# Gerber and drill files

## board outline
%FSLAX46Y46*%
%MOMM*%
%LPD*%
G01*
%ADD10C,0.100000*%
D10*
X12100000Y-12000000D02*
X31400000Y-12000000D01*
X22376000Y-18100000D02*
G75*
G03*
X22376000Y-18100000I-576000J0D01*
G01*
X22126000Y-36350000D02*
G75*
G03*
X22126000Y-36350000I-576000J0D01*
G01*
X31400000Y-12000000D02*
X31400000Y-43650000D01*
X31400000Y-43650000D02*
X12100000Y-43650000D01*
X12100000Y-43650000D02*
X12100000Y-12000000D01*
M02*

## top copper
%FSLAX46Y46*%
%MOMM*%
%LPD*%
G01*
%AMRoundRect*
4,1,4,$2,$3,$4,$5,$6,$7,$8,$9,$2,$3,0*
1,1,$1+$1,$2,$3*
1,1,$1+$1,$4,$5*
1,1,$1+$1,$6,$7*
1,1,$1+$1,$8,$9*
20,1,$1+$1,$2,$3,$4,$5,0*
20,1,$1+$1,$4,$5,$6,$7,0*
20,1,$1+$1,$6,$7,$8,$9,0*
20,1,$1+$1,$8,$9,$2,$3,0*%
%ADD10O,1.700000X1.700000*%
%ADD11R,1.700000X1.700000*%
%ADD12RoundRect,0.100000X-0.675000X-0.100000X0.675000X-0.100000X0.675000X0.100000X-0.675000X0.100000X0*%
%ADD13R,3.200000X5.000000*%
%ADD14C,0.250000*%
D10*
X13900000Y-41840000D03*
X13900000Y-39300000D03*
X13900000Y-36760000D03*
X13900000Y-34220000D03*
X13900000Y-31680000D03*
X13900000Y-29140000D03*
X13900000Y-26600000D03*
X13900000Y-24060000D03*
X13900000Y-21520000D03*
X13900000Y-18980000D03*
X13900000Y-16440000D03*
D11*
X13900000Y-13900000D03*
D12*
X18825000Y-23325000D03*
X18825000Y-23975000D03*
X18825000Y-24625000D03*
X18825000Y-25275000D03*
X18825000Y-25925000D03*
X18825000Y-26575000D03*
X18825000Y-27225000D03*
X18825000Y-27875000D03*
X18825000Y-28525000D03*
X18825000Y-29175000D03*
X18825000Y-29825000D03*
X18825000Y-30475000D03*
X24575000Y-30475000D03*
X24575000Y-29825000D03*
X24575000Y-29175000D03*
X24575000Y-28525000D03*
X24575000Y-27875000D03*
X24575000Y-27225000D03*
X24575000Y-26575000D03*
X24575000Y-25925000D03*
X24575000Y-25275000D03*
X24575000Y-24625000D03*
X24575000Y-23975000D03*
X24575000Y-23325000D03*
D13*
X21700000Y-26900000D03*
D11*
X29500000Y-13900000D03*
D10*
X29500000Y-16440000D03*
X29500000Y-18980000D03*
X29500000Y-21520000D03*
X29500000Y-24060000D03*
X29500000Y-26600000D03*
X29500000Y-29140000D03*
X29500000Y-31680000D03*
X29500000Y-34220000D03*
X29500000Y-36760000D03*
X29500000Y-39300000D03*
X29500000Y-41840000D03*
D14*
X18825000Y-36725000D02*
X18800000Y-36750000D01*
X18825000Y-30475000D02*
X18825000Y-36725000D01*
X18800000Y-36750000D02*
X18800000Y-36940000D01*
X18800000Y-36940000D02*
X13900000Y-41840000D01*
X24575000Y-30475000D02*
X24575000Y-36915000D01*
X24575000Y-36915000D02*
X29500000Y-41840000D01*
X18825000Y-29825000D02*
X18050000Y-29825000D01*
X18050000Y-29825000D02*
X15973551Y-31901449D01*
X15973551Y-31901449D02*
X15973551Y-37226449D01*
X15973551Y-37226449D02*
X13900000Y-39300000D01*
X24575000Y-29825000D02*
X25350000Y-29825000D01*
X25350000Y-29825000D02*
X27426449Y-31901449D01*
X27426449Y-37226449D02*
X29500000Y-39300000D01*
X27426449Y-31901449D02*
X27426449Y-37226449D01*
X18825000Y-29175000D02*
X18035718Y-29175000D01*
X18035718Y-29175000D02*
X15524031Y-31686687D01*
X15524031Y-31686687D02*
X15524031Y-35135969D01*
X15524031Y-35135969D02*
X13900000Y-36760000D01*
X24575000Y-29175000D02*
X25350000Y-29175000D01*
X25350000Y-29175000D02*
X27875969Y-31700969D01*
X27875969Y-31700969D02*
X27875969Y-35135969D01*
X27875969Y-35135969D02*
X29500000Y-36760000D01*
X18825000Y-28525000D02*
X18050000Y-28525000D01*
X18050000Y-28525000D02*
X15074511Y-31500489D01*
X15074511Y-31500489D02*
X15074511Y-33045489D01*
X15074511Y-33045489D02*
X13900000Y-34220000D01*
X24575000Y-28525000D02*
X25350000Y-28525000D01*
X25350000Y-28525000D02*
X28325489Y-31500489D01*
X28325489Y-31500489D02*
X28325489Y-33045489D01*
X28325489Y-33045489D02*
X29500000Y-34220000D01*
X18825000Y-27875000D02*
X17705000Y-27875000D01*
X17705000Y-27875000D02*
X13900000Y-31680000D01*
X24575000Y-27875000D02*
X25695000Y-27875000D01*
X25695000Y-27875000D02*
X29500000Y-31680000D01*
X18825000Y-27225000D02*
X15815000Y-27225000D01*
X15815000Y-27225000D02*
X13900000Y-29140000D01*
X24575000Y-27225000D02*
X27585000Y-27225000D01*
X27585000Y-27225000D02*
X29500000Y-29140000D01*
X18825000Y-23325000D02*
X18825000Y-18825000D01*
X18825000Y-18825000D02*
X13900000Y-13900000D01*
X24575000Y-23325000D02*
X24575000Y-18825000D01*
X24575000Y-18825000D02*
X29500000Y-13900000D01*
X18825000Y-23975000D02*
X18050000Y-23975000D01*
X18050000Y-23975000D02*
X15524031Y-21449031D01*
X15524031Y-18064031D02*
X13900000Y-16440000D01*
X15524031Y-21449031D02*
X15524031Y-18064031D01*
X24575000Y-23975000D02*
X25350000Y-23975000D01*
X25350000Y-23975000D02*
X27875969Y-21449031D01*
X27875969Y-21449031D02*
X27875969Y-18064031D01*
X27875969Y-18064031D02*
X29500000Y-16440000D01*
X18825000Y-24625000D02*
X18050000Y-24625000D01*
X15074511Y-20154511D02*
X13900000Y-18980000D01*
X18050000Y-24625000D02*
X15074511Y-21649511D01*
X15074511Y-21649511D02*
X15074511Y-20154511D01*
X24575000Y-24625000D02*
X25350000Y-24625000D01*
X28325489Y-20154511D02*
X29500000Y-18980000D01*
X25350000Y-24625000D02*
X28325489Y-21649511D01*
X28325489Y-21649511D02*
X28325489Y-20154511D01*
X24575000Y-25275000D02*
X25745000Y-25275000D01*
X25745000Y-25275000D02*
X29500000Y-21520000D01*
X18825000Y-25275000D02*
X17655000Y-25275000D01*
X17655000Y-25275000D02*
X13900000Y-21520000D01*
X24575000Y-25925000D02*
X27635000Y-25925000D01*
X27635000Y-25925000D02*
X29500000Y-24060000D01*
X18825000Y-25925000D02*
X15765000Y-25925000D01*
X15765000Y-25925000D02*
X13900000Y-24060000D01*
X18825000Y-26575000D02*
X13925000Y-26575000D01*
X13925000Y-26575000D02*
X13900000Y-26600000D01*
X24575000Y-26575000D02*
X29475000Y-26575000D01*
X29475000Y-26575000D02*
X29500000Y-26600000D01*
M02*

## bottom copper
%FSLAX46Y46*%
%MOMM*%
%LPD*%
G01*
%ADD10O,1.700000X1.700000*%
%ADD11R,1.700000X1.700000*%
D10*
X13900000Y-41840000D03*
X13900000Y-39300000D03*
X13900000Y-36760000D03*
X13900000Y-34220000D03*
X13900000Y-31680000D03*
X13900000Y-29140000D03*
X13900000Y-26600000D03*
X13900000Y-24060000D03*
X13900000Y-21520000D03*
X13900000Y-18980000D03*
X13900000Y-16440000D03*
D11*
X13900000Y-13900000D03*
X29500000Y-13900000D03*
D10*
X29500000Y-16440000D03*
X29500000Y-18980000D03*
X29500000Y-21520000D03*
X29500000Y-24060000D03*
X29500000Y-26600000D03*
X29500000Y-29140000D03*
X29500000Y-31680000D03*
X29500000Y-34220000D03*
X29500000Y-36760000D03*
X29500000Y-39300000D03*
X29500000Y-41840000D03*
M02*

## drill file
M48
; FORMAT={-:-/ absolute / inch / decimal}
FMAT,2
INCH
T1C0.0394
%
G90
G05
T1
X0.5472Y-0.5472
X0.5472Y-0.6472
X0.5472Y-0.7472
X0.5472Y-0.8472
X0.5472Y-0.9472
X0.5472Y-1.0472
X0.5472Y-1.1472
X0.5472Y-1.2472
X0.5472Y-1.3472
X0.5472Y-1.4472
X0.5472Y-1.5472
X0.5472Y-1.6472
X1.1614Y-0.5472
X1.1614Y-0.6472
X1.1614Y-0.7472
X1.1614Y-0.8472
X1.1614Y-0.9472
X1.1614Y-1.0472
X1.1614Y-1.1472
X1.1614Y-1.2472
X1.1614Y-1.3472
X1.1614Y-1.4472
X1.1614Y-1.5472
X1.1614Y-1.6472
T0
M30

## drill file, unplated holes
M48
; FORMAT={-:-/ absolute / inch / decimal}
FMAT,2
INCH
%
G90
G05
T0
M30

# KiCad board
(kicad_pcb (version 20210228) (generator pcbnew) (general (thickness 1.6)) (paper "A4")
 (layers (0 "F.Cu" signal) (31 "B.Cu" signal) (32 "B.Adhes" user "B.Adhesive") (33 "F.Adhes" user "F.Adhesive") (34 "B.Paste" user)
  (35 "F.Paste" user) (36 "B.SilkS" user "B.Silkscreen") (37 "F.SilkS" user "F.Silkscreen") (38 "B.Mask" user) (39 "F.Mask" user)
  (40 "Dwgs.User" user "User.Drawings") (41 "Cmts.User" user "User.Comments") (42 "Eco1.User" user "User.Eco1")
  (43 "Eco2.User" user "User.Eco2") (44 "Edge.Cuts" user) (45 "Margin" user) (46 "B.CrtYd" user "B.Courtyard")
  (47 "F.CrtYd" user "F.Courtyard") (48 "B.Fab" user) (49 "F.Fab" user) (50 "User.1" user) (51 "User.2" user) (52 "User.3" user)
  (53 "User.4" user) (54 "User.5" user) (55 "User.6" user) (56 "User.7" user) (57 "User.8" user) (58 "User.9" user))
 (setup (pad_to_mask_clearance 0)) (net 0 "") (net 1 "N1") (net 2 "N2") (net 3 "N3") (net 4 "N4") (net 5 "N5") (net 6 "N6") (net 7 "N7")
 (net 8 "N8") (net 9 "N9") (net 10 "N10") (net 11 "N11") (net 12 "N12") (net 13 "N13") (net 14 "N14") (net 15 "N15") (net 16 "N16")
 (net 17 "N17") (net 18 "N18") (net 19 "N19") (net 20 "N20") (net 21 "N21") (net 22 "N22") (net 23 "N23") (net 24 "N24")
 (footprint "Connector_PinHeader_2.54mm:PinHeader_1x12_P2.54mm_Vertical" (layer "F.Cu") (at 13.9 13.9)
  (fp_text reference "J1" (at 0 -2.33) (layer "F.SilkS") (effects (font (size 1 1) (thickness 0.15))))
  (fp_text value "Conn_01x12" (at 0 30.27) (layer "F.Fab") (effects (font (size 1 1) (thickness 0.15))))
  (pad "1" thru_hole rect (at 0 0) (locked) (size 1.7 1.7) (drill 1) (layers *.Cu *.Mask) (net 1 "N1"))
  (pad "2" thru_hole oval (at 0 2.54) (locked) (size 1.7 1.7) (drill 1) (layers *.Cu *.Mask) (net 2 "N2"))
  (pad "3" thru_hole oval (at 0 5.08) (locked) (size 1.7 1.7) (drill 1) (layers *.Cu *.Mask) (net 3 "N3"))
  (pad "4" thru_hole oval (at 0 7.62) (locked) (size 1.7 1.7) (drill 1) (layers *.Cu *.Mask) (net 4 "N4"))
  (pad "5" thru_hole oval (at 0 10.16) (locked) (size 1.7 1.7) (drill 1) (layers *.Cu *.Mask) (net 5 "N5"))
  (pad "6" thru_hole oval (at 0 12.7) (locked) (size 1.7 1.7) (drill 1) (layers *.Cu *.Mask) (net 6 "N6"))
  (pad "7" thru_hole oval (at 0 15.24) (locked) (size 1.7 1.7) (drill 1) (layers *.Cu *.Mask) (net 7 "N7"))
  (pad "8" thru_hole oval (at 0 17.78) (locked) (size 1.7 1.7) (drill 1) (layers *.Cu *.Mask) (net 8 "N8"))
  (pad "9" thru_hole oval (at 0 20.32) (locked) (size 1.7 1.7) (drill 1) (layers *.Cu *.Mask) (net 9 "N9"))
  (pad "10" thru_hole oval (at 0 22.86) (locked) (size 1.7 1.7) (drill 1) (layers *.Cu *.Mask) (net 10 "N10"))
  (pad "11" thru_hole oval (at 0 25.4) (locked) (size 1.7 1.7) (drill 1) (layers *.Cu *.Mask) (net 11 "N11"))
  (pad "12" thru_hole oval (at 0 27.94) (locked) (size 1.7 1.7) (drill 1) (layers *.Cu *.Mask) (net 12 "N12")))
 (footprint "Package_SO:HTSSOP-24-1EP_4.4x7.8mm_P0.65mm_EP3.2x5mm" (layer "F.Cu") (at 21.7 26.9)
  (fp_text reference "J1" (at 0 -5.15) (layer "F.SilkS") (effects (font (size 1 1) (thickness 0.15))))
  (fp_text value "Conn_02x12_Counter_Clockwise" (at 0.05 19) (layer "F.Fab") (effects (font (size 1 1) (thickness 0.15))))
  (pad "" smd roundrect (at -0.8 1.67) (locked) (size 1.29 1.34) (layers "F.Paste") (roundrect_rratio 0.1937976744))
  (pad "" smd roundrect (at 0.8 0) (locked) (size 1.29 1.34) (layers "F.Paste") (roundrect_rratio 0.1937976744))
  (pad "" smd roundrect (at -0.8 -1.67) (locked) (size 1.29 1.34) (layers "F.Paste") (roundrect_rratio 0.1937976744))
  (pad "" smd roundrect (at 0.8 -1.67) (locked) (size 1.29 1.34) (layers "F.Paste") (roundrect_rratio 0.1937976744))
  (pad "" smd roundrect (at -0.8 0) (locked) (size 1.29 1.34) (layers "F.Paste") (roundrect_rratio 0.1937976744))
  (pad "" smd roundrect (at 0.8 1.67) (locked) (size 1.29 1.34) (layers "F.Paste") (roundrect_rratio 0.1937976744))
  (pad "1" smd roundrect (at -2.875 -3.575) (locked) (size 1.55 0.4) (layers "F.Cu" "F.Paste" "F.Mask") (roundrect_rratio 0.25) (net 1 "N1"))
  (pad "2" smd roundrect (at -2.875 -2.925) (locked) (size 1.55 0.4) (layers "F.Cu" "F.Paste" "F.Mask") (roundrect_rratio 0.25) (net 2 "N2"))
  (pad "3" smd roundrect (at -2.875 -2.275) (locked) (size 1.55 0.4) (layers "F.Cu" "F.Paste" "F.Mask") (roundrect_rratio 0.25) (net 3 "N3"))
  (pad "4" smd roundrect (at -2.875 -1.625) (locked) (size 1.55 0.4) (layers "F.Cu" "F.Paste" "F.Mask") (roundrect_rratio 0.25) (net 4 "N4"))
  (pad "5" smd roundrect (at -2.875 -0.975) (locked) (size 1.55 0.4) (layers "F.Cu" "F.Paste" "F.Mask") (roundrect_rratio 0.25) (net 5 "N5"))
  (pad "6" smd roundrect (at -2.875 -0.325) (locked) (size 1.55 0.4) (layers "F.Cu" "F.Paste" "F.Mask") (roundrect_rratio 0.25) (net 6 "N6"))
  (pad "7" smd roundrect (at -2.875 0.325) (locked) (size 1.55 0.4) (layers "F.Cu" "F.Paste" "F.Mask") (roundrect_rratio 0.25) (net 7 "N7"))
  (pad "8" smd roundrect (at -2.875 0.975) (locked) (size 1.55 0.4) (layers "F.Cu" "F.Paste" "F.Mask") (roundrect_rratio 0.25) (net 8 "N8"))
  (pad "9" smd roundrect (at -2.875 1.625) (locked) (size 1.55 0.4) (layers "F.Cu" "F.Paste" "F.Mask") (roundrect_rratio 0.25) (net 9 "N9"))
  (pad "10" smd roundrect (at -2.875 2.275) (locked) (size 1.55 0.4) (layers "F.Cu" "F.Paste" "F.Mask") (roundrect_rratio 0.25)
   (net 10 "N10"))
  (pad "11" smd roundrect (at -2.875 2.925) (locked) (size 1.55 0.4) (layers "F.Cu" "F.Paste" "F.Mask") (roundrect_rratio 0.25)
   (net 11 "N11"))
  (pad "12" smd roundrect (at -2.875 3.575) (locked) (size 1.55 0.4) (layers "F.Cu" "F.Paste" "F.Mask") (roundrect_rratio 0.25)
   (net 12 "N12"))
  (pad "13" smd roundrect (at 2.875 3.575) (locked) (size 1.55 0.4) (layers "F.Cu" "F.Paste" "F.Mask") (roundrect_rratio 0.25)
   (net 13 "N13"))
  (pad "14" smd roundrect (at 2.875 2.925) (locked) (size 1.55 0.4) (layers "F.Cu" "F.Paste" "F.Mask") (roundrect_rratio 0.25)
   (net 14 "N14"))
  (pad "15" smd roundrect (at 2.875 2.275) (locked) (size 1.55 0.4) (layers "F.Cu" "F.Paste" "F.Mask") (roundrect_rratio 0.25)
   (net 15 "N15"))
  (pad "16" smd roundrect (at 2.875 1.625) (locked) (size 1.55 0.4) (layers "F.Cu" "F.Paste" "F.Mask") (roundrect_rratio 0.25)
   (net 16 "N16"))
  (pad "17" smd roundrect (at 2.875 0.975) (locked) (size 1.55 0.4) (layers "F.Cu" "F.Paste" "F.Mask") (roundrect_rratio 0.25)
   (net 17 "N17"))
  (pad "18" smd roundrect (at 2.875 0.325) (locked) (size 1.55 0.4) (layers "F.Cu" "F.Paste" "F.Mask") (roundrect_rratio 0.25)
   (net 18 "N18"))
  (pad "19" smd roundrect (at 2.875 -0.325) (locked) (size 1.55 0.4) (layers "F.Cu" "F.Paste" "F.Mask") (roundrect_rratio 0.25)
   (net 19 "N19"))
  (pad "20" smd roundrect (at 2.875 -0.975) (locked) (size 1.55 0.4) (layers "F.Cu" "F.Paste" "F.Mask") (roundrect_rratio 0.25)
   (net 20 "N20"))
  (pad "21" smd roundrect (at 2.875 -1.625) (locked) (size 1.55 0.4) (layers "F.Cu" "F.Paste" "F.Mask") (roundrect_rratio 0.25)
   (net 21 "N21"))
  (pad "22" smd roundrect (at 2.875 -2.275) (locked) (size 1.55 0.4) (layers "F.Cu" "F.Paste" "F.Mask") (roundrect_rratio 0.25)
   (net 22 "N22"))
  (pad "23" smd roundrect (at 2.875 -2.925) (locked) (size 1.55 0.4) (layers "F.Cu" "F.Paste" "F.Mask") (roundrect_rratio 0.25)
   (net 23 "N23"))
  (pad "24" smd roundrect (at 2.875 -3.575) (locked) (size 1.55 0.4) (layers "F.Cu" "F.Paste" "F.Mask") (roundrect_rratio 0.25)
   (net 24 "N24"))
  (pad "25" smd rect (at 0 0) (locked) (size 3.2 5) (layers "F.Cu" "F.Mask")))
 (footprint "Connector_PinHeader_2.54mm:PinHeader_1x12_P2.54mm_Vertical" (layer "F.Cu") (at 29.5 13.9)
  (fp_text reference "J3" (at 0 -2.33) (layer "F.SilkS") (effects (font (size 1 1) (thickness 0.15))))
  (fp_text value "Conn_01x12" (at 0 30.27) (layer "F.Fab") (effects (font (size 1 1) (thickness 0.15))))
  (pad "1" thru_hole rect (at 0 0) (locked) (size 1.7 1.7) (drill 1) (layers *.Cu *.Mask) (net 24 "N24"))
  (pad "2" thru_hole oval (at 0 2.54) (locked) (size 1.7 1.7) (drill 1) (layers *.Cu *.Mask) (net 23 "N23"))
  (pad "3" thru_hole oval (at 0 5.08) (locked) (size 1.7 1.7) (drill 1) (layers *.Cu *.Mask) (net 22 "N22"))
  (pad "4" thru_hole oval (at 0 7.62) (locked) (size 1.7 1.7) (drill 1) (layers *.Cu *.Mask) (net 21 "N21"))
  (pad "5" thru_hole oval (at 0 10.16) (locked) (size 1.7 1.7) (drill 1) (layers *.Cu *.Mask) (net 20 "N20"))
  (pad "6" thru_hole oval (at 0 12.7) (locked) (size 1.7 1.7) (drill 1) (layers *.Cu *.Mask) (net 19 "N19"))
  (pad "7" thru_hole oval (at 0 15.24) (locked) (size 1.7 1.7) (drill 1) (layers *.Cu *.Mask) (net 18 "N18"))
  (pad "8" thru_hole oval (at 0 17.78) (locked) (size 1.7 1.7) (drill 1) (layers *.Cu *.Mask) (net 17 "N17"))
  (pad "9" thru_hole oval (at 0 20.32) (locked) (size 1.7 1.7) (drill 1) (layers *.Cu *.Mask) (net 16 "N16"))
  (pad "10" thru_hole oval (at 0 22.86) (locked) (size 1.7 1.7) (drill 1) (layers *.Cu *.Mask) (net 15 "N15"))
  (pad "11" thru_hole oval (at 0 25.4) (locked) (size 1.7 1.7) (drill 1) (layers *.Cu *.Mask) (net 14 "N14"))
  (pad "12" thru_hole oval (at 0 27.94) (locked) (size 1.7 1.7) (drill 1) (layers *.Cu *.Mask) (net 13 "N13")))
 (gr_line (start 31.4 12) (end 31.4 43.65) (layer "Edge.Cuts") (width 0.1))
 (gr_line (start 12.1 12) (end 31.4 12) (layer "Edge.Cuts") (width 0.1))
 (gr_circle (center 21.8 18.1) (end 22.376 18.1) (layer "Edge.Cuts") (width 0.1) (fill none))
 (gr_line (start 31.4 43.65) (end 12.1 43.65) (layer "Edge.Cuts") (width 0.1))
 (gr_circle (center 21.55 36.35) (end 22.126 36.35) (layer "Edge.Cuts") (width 0.1) (fill none))
 (gr_line (start 12.1 43.65) (end 12.1 12) (layer "Edge.Cuts") (width 0.1))
 (segment (start 18.825 18.825) (end 13.9 13.9) (width 0.25) (layer "F.Cu") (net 1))
 (segment (start 18.825 23.325) (end 18.825 18.825) (width 0.25) (layer "F.Cu") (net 1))
 (segment (start 18.825 23.975) (end 18.05 23.975) (width 0.25) (layer "F.Cu") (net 2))
 (segment (start 18.05 23.975) (end 15.524031 21.449031) (width 0.25) (layer "F.Cu") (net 2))
 (segment (start 15.524031 18.064031) (end 13.9 16.44) (width 0.25) (layer "F.Cu") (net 2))
 (segment (start 15.524031 21.449031) (end 15.524031 18.064031) (width 0.25) (layer "F.Cu") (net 2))
 (segment (start 15.074511 20.154511) (end 13.9 18.98) (width 0.25) (layer "F.Cu") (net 3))
 (segment (start 15.074511 21.649511) (end 15.074511 20.154511) (width 0.25) (layer "F.Cu") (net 3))
 (segment (start 18.825 24.625) (end 18.05 24.625) (width 0.25) (layer "F.Cu") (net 3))
 (segment (start 18.05 24.625) (end 15.074511 21.649511) (width 0.25) (layer "F.Cu") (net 3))
 (segment (start 17.655 25.275) (end 13.9 21.52) (width 0.25) (layer "F.Cu") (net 4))
 (segment (start 18.825 25.275) (end 17.655 25.275) (width 0.25) (layer "F.Cu") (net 4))
 (segment (start 18.825 25.925) (end 15.765 25.925) (width 0.25) (layer "F.Cu") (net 5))
 (segment (start 15.765 25.925) (end 13.9 24.06) (width 0.25) (layer "F.Cu") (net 5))
 (segment (start 13.925 26.575) (end 13.9 26.6) (width 0.25) (layer "F.Cu") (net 6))
 (segment (start 18.825 26.575) (end 13.925 26.575) (width 0.25) (layer "F.Cu") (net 6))
 (segment (start 18.825 27.225) (end 15.815 27.225) (width 0.25) (layer "F.Cu") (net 7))
 (segment (start 15.815 27.225) (end 13.9 29.14) (width 0.25) (layer "F.Cu") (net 7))
 (segment (start 18.825 27.875) (end 17.705 27.875) (width 0.25) (layer "F.Cu") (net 8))
 (segment (start 17.705 27.875) (end 13.9 31.68) (width 0.25) (layer "F.Cu") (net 8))
 (segment (start 18.825 28.525) (end 18.05 28.525) (width 0.25) (layer "F.Cu") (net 9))
 (segment (start 15.074511 33.045489) (end 13.9 34.22) (width 0.25) (layer "F.Cu") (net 9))
 (segment (start 18.05 28.525) (end 15.074511 31.500489) (width 0.25) (layer "F.Cu") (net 9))
 (segment (start 15.074511 31.500489) (end 15.074511 33.045489) (width 0.25) (layer "F.Cu") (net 9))
 (segment (start 18.825 29.175) (end 18.035718 29.175) (width 0.25) (layer "F.Cu") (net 10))
 (segment (start 15.524031 35.135969) (end 13.9 36.76) (width 0.25) (layer "F.Cu") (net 10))
 (segment (start 15.524031 31.686687) (end 15.524031 35.135969) (width 0.25) (layer "F.Cu") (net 10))
 (segment (start 18.035718 29.175) (end 15.524031 31.686687) (width 0.25) (layer "F.Cu") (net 10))
 (segment (start 18.825 29.825) (end 18.05 29.825) (width 0.25) (layer "F.Cu") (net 11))
 (segment (start 15.973551 37.226449) (end 13.9 39.3) (width 0.25) (layer "F.Cu") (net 11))
 (segment (start 15.973551 31.901449) (end 15.973551 37.226449) (width 0.25) (layer "F.Cu") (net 11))
 (segment (start 18.05 29.825) (end 15.973551 31.901449) (width 0.25) (layer "F.Cu") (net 11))
 (segment (start 18.8 36.94) (end 13.9 41.84) (width 0.25) (layer "F.Cu") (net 12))
 (segment (start 18.825 30.475) (end 18.825 36.725) (width 0.25) (layer "F.Cu") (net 12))
 (segment (start 18.8 36.75) (end 18.8 36.94) (width 0.25) (layer "F.Cu") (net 12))
 (segment (start 18.825 36.725) (end 18.8 36.75) (width 0.25) (layer "F.Cu") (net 12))
 (segment (start 24.575 30.475) (end 24.575 36.915) (width 0.25) (layer "F.Cu") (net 13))
 (segment (start 24.575 36.915) (end 29.5 41.84) (width 0.25) (layer "F.Cu") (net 13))
 (segment (start 27.426449 31.901449) (end 27.426449 37.226449) (width 0.25) (layer "F.Cu") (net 14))
 (segment (start 24.575 29.825) (end 25.35 29.825) (width 0.25) (layer "F.Cu") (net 14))
 (segment (start 27.426449 37.226449) (end 29.5 39.3) (width 0.25) (layer "F.Cu") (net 14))
 (segment (start 25.35 29.825) (end 27.426449 31.901449) (width 0.25) (layer "F.Cu") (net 14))
 (segment (start 25.35 29.175) (end 27.875969 31.700969) (width 0.25) (layer "F.Cu") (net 15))
 (segment (start 24.575 29.175) (end 25.35 29.175) (width 0.25) (layer "F.Cu") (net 15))
 (segment (start 27.875969 35.135969) (end 29.5 36.76) (width 0.25) (layer "F.Cu") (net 15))
 (segment (start 27.875969 31.700969) (end 27.875969 35.135969) (width 0.25) (layer "F.Cu") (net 15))
 (segment (start 28.325489 31.500489) (end 28.325489 33.045489) (width 0.25) (layer "F.Cu") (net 16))
 (segment (start 28.325489 33.045489) (end 29.5 34.22) (width 0.25) (layer "F.Cu") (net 16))
 (segment (start 24.575 28.525) (end 25.35 28.525) (width 0.25) (layer "F.Cu") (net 16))
 (segment (start 25.35 28.525) (end 28.325489 31.500489) (width 0.25) (layer "F.Cu") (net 16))
 (segment (start 25.695 27.875) (end 29.5 31.68) (width 0.25) (layer "F.Cu") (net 17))
 (segment (start 24.575 27.875) (end 25.695 27.875) (width 0.25) (layer "F.Cu") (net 17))
 (segment (start 24.575 27.225) (end 27.585 27.225) (width 0.25) (layer "F.Cu") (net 18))
 (segment (start 27.585 27.225) (end 29.5 29.14) (width 0.25) (layer "F.Cu") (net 18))
 (segment (start 29.475 26.575) (end 29.5 26.6) (width 0.25) (layer "F.Cu") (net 19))
 (segment (start 24.575 26.575) (end 29.475 26.575) (width 0.25) (layer "F.Cu") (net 19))
 (segment (start 24.575 25.925) (end 27.635 25.925) (width 0.25) (layer "F.Cu") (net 20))
 (segment (start 27.635 25.925) (end 29.5 24.06) (width 0.25) (layer "F.Cu") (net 20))
 (segment (start 24.575 25.275) (end 25.745 25.275) (width 0.25) (layer "F.Cu") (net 21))
 (segment (start 25.745 25.275) (end 29.5 21.52) (width 0.25) (layer "F.Cu") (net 21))
 (segment (start 28.325489 21.649511) (end 28.325489 20.154511) (width 0.25) (layer "F.Cu") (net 22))
 (segment (start 24.575 24.625) (end 25.35 24.625) (width 0.25) (layer "F.Cu") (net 22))
 (segment (start 28.325489 20.154511) (end 29.5 18.98) (width 0.25) (layer "F.Cu") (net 22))
 (segment (start 25.35 24.625) (end 28.325489 21.649511) (width 0.25) (layer "F.Cu") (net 22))
 (segment (start 25.35 23.975) (end 27.875969 21.449031) (width 0.25) (layer "F.Cu") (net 23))
 (segment (start 27.875969 21.449031) (end 27.875969 18.064031) (width 0.25) (layer "F.Cu") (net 23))
 (segment (start 27.875969 18.064031) (end 29.5 16.44) (width 0.25) (layer "F.Cu") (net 23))
 (segment (start 24.575 23.975) (end 25.35 23.975) (width 0.25) (layer "F.Cu") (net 23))
 (segment (start 24.575 23.325) (end 24.575 18.825) (width 0.25) (layer "F.Cu") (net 24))
 (segment (start 24.575 18.825) (end 29.5 13.9) (width 0.25) (layer "F.Cu") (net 24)))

